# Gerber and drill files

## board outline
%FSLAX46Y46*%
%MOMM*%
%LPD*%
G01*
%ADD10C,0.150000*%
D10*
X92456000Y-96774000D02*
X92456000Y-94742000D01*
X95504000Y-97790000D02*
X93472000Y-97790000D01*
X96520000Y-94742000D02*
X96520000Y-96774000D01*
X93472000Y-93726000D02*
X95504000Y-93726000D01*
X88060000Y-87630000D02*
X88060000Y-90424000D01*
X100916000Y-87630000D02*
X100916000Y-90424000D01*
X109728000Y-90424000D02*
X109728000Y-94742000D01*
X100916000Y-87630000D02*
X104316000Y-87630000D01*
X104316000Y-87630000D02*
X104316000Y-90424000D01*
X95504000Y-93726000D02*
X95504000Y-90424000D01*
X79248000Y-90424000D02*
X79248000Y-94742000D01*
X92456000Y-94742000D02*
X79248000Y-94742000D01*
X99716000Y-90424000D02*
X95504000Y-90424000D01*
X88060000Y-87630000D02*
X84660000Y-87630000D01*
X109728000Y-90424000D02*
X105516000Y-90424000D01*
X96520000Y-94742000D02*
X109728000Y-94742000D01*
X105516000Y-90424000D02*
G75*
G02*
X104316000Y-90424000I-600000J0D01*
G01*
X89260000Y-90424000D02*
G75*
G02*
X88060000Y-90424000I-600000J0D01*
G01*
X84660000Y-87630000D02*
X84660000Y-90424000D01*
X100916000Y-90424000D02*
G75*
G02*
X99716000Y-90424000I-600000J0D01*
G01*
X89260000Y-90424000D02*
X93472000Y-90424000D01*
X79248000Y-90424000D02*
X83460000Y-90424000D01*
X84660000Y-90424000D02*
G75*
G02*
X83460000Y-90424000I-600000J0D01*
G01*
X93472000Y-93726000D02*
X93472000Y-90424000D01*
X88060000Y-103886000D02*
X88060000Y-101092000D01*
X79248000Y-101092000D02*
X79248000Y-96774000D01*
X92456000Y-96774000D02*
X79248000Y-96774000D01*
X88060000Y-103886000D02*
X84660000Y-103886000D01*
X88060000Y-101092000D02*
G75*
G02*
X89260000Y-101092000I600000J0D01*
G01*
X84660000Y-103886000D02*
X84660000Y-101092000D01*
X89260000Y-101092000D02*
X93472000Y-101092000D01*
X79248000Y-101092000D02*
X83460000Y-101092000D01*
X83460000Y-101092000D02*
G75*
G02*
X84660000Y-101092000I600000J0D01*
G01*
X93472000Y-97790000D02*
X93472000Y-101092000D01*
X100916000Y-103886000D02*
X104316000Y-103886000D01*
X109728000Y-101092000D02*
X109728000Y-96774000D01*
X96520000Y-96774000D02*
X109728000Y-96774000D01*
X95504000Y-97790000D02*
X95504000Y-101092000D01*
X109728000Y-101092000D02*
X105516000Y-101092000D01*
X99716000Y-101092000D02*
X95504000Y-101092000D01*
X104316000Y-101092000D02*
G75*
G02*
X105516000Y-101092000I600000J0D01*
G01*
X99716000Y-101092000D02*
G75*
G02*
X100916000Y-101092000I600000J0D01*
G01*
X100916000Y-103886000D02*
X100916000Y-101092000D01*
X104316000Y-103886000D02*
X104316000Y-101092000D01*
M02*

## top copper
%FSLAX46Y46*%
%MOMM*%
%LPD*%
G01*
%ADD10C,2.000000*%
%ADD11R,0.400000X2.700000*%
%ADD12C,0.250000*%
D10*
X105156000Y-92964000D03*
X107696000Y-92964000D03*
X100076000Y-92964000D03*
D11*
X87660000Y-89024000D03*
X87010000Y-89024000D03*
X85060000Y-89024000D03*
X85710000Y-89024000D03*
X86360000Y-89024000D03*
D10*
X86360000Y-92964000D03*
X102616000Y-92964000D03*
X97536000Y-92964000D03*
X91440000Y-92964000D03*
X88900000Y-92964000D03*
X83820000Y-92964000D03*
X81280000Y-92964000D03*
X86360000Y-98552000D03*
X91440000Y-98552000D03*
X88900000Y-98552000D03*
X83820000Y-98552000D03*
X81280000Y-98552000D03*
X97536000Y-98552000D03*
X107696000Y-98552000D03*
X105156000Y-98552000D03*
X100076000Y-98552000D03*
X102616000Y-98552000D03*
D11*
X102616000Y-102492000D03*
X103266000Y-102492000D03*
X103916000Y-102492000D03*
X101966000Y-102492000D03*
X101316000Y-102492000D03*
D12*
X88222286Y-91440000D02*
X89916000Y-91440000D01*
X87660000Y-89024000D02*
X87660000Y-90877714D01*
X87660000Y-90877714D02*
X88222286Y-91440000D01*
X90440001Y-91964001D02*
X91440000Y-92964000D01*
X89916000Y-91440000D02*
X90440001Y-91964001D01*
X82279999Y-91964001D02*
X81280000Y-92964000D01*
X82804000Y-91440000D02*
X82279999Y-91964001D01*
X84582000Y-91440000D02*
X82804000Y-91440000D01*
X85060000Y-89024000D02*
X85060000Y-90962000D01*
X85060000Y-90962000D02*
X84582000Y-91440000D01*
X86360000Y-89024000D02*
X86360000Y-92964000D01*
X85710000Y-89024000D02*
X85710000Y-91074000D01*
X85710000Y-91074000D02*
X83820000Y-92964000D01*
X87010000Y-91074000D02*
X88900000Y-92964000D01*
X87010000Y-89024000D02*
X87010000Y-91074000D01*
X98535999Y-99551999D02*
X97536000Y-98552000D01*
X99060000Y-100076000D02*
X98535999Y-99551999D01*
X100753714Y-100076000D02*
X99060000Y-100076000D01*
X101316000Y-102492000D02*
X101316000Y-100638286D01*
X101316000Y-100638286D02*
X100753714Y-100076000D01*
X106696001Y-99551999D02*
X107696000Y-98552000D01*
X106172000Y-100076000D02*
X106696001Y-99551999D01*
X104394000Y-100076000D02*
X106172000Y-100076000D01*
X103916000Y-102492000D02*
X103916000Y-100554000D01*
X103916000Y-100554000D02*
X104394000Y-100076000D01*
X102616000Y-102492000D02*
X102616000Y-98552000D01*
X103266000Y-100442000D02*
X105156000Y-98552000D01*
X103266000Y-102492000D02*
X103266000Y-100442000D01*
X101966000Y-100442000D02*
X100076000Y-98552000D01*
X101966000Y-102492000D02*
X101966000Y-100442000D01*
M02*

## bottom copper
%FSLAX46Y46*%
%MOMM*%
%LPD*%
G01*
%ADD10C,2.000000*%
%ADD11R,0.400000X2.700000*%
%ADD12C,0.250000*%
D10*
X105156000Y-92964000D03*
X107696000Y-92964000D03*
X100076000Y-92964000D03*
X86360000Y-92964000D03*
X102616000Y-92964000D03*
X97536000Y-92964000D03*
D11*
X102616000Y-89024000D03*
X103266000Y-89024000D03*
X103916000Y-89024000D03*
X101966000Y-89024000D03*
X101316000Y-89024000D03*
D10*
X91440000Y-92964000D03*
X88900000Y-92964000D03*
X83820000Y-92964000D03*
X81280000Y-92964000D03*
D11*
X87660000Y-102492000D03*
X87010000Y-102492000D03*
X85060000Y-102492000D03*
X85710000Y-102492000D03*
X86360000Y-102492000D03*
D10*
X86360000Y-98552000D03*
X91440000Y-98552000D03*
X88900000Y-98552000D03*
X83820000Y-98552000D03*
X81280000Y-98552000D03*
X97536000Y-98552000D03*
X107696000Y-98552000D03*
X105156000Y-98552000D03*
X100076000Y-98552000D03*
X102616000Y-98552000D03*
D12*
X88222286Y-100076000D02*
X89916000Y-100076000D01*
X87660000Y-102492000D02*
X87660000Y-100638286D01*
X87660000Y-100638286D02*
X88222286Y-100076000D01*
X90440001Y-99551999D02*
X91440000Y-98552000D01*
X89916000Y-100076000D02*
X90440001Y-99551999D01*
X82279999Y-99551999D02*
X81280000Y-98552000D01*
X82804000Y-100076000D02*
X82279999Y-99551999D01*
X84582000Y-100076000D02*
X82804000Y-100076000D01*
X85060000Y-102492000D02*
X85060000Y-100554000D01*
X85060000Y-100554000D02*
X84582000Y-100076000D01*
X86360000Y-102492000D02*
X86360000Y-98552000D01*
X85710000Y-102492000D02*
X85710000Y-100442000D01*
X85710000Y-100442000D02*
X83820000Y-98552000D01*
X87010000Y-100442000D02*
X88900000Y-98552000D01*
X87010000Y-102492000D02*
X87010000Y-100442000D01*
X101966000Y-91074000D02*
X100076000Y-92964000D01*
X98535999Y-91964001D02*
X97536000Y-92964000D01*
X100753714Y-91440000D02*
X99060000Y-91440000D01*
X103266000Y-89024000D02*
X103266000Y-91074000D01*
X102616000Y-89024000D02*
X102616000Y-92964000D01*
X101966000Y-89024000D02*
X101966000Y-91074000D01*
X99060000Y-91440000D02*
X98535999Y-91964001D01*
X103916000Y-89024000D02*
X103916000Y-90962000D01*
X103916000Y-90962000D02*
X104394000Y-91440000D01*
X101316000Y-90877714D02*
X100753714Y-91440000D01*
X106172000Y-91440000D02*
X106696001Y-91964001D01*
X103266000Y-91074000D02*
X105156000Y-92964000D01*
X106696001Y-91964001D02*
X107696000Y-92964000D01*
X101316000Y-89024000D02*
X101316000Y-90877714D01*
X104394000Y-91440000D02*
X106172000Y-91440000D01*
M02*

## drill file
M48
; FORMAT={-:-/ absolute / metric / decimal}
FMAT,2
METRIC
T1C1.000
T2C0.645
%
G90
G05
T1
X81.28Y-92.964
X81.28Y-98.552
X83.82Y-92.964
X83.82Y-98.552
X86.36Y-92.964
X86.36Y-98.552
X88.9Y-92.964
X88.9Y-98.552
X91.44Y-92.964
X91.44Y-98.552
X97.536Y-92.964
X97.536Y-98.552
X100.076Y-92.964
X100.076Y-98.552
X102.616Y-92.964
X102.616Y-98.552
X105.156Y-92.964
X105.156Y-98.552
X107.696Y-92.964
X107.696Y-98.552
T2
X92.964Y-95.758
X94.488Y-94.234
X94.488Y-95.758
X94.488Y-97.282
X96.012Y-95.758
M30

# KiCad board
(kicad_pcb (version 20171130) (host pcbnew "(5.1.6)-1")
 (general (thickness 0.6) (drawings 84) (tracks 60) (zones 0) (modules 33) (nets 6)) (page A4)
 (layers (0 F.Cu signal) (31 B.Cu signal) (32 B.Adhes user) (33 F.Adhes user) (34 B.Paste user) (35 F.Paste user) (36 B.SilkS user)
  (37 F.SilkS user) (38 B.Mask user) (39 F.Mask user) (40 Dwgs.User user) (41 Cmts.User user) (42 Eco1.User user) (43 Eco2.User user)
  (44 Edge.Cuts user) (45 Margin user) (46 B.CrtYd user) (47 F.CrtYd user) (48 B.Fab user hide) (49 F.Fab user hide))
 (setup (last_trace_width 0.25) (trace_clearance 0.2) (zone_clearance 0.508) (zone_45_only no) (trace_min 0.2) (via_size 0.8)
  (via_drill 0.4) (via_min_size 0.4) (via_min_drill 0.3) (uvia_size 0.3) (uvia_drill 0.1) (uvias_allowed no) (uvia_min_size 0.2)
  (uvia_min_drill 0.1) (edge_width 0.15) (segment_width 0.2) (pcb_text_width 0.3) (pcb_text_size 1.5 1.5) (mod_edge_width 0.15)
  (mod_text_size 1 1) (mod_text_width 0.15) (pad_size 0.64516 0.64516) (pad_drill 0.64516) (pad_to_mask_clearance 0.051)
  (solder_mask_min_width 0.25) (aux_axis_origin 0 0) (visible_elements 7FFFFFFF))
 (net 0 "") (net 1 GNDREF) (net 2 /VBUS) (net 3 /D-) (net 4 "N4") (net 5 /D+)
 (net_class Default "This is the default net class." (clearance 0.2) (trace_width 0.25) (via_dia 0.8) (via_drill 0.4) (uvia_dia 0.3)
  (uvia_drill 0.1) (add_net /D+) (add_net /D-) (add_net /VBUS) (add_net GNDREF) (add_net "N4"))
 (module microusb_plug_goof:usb (layer B.Cu) (at 86.3364 88.9 180)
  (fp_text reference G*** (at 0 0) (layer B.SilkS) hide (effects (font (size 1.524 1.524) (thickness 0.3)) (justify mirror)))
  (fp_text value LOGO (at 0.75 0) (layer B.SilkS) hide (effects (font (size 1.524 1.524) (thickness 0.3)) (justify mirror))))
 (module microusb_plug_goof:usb (layer F.Cu) (at 102.6396 88.9)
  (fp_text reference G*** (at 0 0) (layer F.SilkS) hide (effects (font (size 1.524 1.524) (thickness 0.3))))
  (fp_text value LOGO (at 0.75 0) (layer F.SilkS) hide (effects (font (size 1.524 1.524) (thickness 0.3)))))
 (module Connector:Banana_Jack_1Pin (layer F.Cu) (at 94.488 97.282)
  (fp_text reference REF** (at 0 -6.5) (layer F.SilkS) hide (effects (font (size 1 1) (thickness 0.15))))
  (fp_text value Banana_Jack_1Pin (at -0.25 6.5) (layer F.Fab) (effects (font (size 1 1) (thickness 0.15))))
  (pad "" np_thru_hole circle (at 0 0) (size 0.64516 0.64516) (drill 0.64516) (layers *.Cu *.Mask)))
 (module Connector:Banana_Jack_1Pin (layer F.Cu) (at 94.488 94.234)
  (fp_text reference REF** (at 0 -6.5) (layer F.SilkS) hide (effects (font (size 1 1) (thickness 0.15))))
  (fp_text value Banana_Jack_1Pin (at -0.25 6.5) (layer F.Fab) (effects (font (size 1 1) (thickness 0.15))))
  (pad "" np_thru_hole circle (at 0 0) (size 0.64516 0.64516) (drill 0.64516) (layers *.Cu *.Mask)))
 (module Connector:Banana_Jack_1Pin (layer F.Cu) (at 96.012 95.758)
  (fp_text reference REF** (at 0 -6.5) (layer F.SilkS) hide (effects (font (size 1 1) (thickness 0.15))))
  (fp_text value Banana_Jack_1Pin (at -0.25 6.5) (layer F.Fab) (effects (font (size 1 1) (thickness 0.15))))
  (pad "" np_thru_hole circle (at 0 0) (size 0.64516 0.64516) (drill 0.64516) (layers *.Cu *.Mask)))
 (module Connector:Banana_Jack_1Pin (layer F.Cu) (at 92.964 95.758)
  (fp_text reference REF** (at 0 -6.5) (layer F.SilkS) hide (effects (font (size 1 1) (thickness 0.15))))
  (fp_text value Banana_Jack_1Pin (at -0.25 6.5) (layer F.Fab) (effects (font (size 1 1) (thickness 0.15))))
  (pad "" np_thru_hole circle (at 0 0) (size 0.64516 0.64516) (drill 0.64516) (layers *.Cu *.Mask)))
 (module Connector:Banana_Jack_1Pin (layer F.Cu) (at 94.488 95.758)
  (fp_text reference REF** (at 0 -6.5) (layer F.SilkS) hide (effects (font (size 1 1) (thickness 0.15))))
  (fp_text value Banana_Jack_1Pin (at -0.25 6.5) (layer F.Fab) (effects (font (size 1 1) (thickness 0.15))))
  (pad "" np_thru_hole circle (at 0 0) (size 0.64516 0.64516) (drill 0.64516) (layers *.Cu *.Mask)))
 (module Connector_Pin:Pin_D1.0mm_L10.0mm (layer B.Cu) (at 105.156 92.964)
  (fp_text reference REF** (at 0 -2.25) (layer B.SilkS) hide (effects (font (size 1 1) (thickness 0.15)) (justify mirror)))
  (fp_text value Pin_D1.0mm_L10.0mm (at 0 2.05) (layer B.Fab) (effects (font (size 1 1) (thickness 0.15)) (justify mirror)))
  (pad 1 thru_hole circle (at 0 0) (size 2 2) (drill 1) (layers *.Cu *.Mask)))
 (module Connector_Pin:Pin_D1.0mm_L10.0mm (layer B.Cu) (at 107.696 92.964)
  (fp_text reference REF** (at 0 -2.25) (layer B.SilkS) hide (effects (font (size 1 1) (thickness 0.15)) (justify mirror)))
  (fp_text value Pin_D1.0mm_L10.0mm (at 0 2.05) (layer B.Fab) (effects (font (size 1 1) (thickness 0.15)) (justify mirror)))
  (pad 1 thru_hole circle (at 0 0) (size 2 2) (drill 1) (layers *.Cu *.Mask)))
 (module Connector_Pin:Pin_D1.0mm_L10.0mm (layer B.Cu) (at 100.076 92.964)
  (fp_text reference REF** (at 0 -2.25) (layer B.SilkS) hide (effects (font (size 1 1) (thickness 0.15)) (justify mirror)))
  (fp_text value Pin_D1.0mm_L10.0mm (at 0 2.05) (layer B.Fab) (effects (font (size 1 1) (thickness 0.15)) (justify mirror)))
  (pad 1 thru_hole circle (at 0 0) (size 2 2) (drill 1) (layers *.Cu *.Mask)))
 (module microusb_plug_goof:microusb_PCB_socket (layer F.Cu) (at 86.36 89.024)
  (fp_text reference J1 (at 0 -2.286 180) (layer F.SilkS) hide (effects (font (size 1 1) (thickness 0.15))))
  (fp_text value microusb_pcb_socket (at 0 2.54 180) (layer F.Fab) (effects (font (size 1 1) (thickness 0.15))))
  (pad 5 smd rect (at 1.3 0) (size 0.4 2.7) (layers F.Cu F.Paste F.Mask))
  (pad 4 smd rect (at 0.65 0) (size 0.4 2.7) (layers F.Cu F.Paste F.Mask))
  (pad 1 smd rect (at -1.3 0) (size 0.4 2.7) (layers F.Cu F.Paste F.Mask))
  (pad 2 smd rect (at -0.65 0) (size 0.4 2.7) (layers F.Cu F.Paste F.Mask))
  (pad 3 smd rect (at 0 0) (size 0.4 2.7) (layers F.Cu F.Paste F.Mask)))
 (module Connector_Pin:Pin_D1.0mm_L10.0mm (layer F.Cu) (at 86.36 92.964 180)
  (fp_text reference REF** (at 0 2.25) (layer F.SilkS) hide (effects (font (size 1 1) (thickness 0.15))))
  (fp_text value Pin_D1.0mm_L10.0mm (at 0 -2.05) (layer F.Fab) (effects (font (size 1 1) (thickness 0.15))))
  (pad 1 thru_hole circle (at 0 0 180) (size 2 2) (drill 1) (layers *.Cu *.Mask)))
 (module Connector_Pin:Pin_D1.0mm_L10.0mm (layer B.Cu) (at 102.616 92.964)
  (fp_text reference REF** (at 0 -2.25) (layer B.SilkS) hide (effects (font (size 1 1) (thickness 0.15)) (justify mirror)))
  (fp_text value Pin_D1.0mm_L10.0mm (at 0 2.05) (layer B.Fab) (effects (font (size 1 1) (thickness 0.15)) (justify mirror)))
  (pad 1 thru_hole circle (at 0 0) (size 2 2) (drill 1) (layers *.Cu *.Mask)))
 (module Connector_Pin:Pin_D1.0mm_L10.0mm (layer B.Cu) (at 97.536 92.964)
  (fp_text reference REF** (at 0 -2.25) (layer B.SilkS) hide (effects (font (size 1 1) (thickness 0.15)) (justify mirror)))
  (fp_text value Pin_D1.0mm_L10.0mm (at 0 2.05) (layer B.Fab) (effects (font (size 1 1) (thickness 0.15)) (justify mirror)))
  (pad 1 thru_hole circle (at 0 0) (size 2 2) (drill 1) (layers *.Cu *.Mask)))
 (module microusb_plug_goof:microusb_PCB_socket (layer B.Cu) (at 102.616 89.024 180)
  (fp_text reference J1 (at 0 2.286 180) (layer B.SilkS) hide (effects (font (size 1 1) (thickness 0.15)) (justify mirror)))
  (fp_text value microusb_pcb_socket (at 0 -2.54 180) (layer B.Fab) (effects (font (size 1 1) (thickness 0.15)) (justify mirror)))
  (pad 3 smd rect (at 0 0 180) (size 0.4 2.7) (layers B.Cu B.Paste B.Mask))
  (pad 2 smd rect (at -0.65 0 180) (size 0.4 2.7) (layers B.Cu B.Paste B.Mask))
  (pad 1 smd rect (at -1.3 0 180) (size 0.4 2.7) (layers B.Cu B.Paste B.Mask))
  (pad 4 smd rect (at 0.65 0 180) (size 0.4 2.7) (layers B.Cu B.Paste B.Mask))
  (pad 5 smd rect (at 1.3 0 180) (size 0.4 2.7) (layers B.Cu B.Paste B.Mask)))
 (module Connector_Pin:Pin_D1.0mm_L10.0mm (layer F.Cu) (at 91.44 92.964 180)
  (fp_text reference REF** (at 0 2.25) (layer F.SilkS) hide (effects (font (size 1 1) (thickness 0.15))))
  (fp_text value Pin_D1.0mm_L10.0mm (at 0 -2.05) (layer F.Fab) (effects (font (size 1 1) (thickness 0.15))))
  (pad 1 thru_hole circle (at 0 0 180) (size 2 2) (drill 1) (layers *.Cu *.Mask)))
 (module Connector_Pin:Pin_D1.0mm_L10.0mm (layer F.Cu) (at 88.9 92.964 180)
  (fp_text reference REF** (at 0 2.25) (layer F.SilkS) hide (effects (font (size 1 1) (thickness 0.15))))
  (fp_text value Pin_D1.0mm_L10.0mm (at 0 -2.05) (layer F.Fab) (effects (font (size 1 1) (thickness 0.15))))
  (pad 1 thru_hole circle (at 0 0 180) (size 2 2) (drill 1) (layers *.Cu *.Mask)))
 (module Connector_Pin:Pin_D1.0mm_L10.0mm (layer F.Cu) (at 83.82 92.964 180)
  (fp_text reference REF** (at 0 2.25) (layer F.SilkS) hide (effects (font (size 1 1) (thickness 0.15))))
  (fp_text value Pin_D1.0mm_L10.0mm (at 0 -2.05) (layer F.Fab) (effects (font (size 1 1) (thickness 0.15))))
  (pad 1 thru_hole circle (at 0 0 180) (size 2 2) (drill 1) (layers *.Cu *.Mask)))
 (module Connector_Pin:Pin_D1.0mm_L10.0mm (layer F.Cu) (at 81.28 92.964 180)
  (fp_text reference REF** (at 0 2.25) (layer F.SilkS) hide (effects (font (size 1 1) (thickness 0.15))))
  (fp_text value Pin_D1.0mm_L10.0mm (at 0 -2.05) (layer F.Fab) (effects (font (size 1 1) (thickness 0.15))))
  (pad 1 thru_hole circle (at 0 0 180) (size 2 2) (drill 1) (layers *.Cu *.Mask)))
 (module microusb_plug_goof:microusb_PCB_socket (layer B.Cu) (at 86.36 102.492)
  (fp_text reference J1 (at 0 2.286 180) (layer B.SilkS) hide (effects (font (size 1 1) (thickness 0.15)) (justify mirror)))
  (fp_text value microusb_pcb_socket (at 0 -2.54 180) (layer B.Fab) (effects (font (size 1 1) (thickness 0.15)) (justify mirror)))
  (pad 5 smd rect (at 1.3 0) (size 0.4 2.7) (layers B.Cu B.Paste B.Mask))
  (pad 4 smd rect (at 0.65 0) (size 0.4 2.7) (layers B.Cu B.Paste B.Mask))
  (pad 1 smd rect (at -1.3 0) (size 0.4 2.7) (layers B.Cu B.Paste B.Mask))
  (pad 2 smd rect (at -0.65 0) (size 0.4 2.7) (layers B.Cu B.Paste B.Mask))
  (pad 3 smd rect (at 0 0) (size 0.4 2.7) (layers B.Cu B.Paste B.Mask)))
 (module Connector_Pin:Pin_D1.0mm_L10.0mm (layer B.Cu) (at 86.36 98.552 180)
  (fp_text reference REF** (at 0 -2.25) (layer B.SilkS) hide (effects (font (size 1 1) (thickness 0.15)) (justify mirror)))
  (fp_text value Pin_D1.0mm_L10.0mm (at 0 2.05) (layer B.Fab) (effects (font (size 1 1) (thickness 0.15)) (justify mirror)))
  (pad 1 thru_hole circle (at 0 0 180) (size 2 2) (drill 1) (layers *.Cu *.Mask)))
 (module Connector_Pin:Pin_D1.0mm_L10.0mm (layer B.Cu) (at 91.44 98.552 180)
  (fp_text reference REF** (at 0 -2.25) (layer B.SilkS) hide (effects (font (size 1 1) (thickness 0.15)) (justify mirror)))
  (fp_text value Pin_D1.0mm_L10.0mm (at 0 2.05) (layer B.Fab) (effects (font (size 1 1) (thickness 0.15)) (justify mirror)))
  (pad 1 thru_hole circle (at 0 0 180) (size 2 2) (drill 1) (layers *.Cu *.Mask)))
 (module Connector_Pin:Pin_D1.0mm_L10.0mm (layer B.Cu) (at 88.9 98.552 180)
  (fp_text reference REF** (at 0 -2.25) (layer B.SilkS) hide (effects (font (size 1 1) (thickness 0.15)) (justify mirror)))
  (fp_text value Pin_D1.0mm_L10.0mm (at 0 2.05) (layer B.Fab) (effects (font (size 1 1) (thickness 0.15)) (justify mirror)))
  (pad 1 thru_hole circle (at 0 0 180) (size 2 2) (drill 1) (layers *.Cu *.Mask)))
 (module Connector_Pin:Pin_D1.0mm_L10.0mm (layer B.Cu) (at 83.82 98.552 180)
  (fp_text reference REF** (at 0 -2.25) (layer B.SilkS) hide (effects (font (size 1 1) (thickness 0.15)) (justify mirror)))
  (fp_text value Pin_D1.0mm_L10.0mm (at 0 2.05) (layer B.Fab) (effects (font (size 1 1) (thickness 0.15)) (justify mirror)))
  (pad 1 thru_hole circle (at 0 0 180) (size 2 2) (drill 1) (layers *.Cu *.Mask)))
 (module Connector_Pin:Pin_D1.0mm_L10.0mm (layer B.Cu) (at 81.28 98.552 180)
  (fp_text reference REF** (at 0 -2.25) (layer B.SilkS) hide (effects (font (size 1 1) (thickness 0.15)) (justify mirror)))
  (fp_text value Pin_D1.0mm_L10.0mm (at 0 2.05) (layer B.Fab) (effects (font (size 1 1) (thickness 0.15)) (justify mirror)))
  (pad 1 thru_hole circle (at 0 0 180) (size 2 2) (drill 1) (layers *.Cu *.Mask)))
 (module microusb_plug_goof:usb (layer F.Cu) (at 86.36 102.616 180)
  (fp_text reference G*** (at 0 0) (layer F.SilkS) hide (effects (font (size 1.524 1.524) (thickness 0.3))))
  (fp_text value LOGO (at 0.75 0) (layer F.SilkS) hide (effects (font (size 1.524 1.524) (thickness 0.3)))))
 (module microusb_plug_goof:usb (layer B.Cu) (at 102.616 102.616)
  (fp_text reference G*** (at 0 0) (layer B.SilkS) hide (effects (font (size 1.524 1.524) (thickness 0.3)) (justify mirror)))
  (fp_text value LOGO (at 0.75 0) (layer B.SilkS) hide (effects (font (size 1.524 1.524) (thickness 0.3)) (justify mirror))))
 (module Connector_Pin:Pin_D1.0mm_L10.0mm (layer F.Cu) (at 97.536 98.552)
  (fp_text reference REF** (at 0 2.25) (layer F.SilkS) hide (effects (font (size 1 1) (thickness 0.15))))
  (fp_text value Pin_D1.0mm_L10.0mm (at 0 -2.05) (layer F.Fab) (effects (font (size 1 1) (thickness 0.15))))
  (pad 1 thru_hole circle (at 0 0) (size 2 2) (drill 1) (layers *.Cu *.Mask) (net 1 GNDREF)))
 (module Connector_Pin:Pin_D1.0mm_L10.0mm (layer F.Cu) (at 107.696 98.552)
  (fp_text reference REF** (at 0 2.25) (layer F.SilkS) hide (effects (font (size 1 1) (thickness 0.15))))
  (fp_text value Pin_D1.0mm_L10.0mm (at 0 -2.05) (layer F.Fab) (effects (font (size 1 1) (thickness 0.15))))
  (pad 1 thru_hole circle (at 0 0) (size 2 2) (drill 1) (layers *.Cu *.Mask) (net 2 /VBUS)))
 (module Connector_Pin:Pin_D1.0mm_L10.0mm (layer F.Cu) (at 105.156 98.552)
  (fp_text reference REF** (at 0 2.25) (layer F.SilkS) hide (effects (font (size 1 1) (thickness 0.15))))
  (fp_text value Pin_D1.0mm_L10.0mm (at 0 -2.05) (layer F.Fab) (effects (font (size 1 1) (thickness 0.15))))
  (pad 1 thru_hole circle (at 0 0) (size 2 2) (drill 1) (layers *.Cu *.Mask) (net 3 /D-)))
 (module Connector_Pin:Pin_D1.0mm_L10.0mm (layer F.Cu) (at 100.076 98.552)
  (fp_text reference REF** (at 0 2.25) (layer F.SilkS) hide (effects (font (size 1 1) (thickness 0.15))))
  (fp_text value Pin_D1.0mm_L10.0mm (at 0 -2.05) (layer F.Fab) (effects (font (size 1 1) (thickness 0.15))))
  (pad 1 thru_hole circle (at 0 0) (size 2 2) (drill 1) (layers *.Cu *.Mask) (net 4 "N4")))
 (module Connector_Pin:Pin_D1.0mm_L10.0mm (layer F.Cu) (at 102.616 98.552)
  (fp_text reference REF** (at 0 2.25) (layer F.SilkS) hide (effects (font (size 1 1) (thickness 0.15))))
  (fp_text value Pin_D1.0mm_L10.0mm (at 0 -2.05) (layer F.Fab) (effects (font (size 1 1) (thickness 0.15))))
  (pad 1 thru_hole circle (at 0 0) (size 2 2) (drill 1) (layers *.Cu *.Mask) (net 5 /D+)))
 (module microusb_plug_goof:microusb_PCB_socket (layer F.Cu) (at 102.616 102.492 180)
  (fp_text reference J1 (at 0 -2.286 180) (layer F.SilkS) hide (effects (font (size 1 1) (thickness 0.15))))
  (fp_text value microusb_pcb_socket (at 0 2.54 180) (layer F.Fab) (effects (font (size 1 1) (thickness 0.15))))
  (pad 3 smd rect (at 0 0 180) (size 0.4 2.7) (layers F.Cu F.Paste F.Mask) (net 5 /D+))
  (pad 2 smd rect (at -0.65 0 180) (size 0.4 2.7) (layers F.Cu F.Paste F.Mask) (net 3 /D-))
  (pad 1 smd rect (at -1.3 0 180) (size 0.4 2.7) (layers F.Cu F.Paste F.Mask) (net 2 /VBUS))
  (pad 4 smd rect (at 0.65 0 180) (size 0.4 2.7) (layers F.Cu F.Paste F.Mask) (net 4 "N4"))
  (pad 5 smd rect (at 1.3 0 180) (size 0.4 2.7) (layers F.Cu F.Paste F.Mask) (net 1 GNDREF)))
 (gr_line (start 92.456 96.774) (end 92.456 94.742) (layer Edge.Cuts) (width 0.15))
 (gr_line (start 95.504 97.79) (end 93.472 97.79) (layer Edge.Cuts) (width 0.15))
 (gr_line (start 96.52 94.742) (end 96.52 96.774) (layer Edge.Cuts) (width 0.15))
 (gr_line (start 93.472 93.726) (end 95.504 93.726) (layer Edge.Cuts) (width 0.15))
 (gr_line (start 88.06 87.63) (end 88.06 90.424) (layer Edge.Cuts) (width 0.15))
 (gr_line (start 100.916 87.63) (end 100.916 90.424) (layer Edge.Cuts) (width 0.15))
 (gr_line (start 109.728 90.424) (end 109.728 94.742) (layer Edge.Cuts) (width 0.15))
 (gr_line (start 100.916 87.63) (end 104.316 87.63) (layer Edge.Cuts) (width 0.15))
 (gr_line (start 104.316 87.63) (end 104.316 90.424) (layer Edge.Cuts) (width 0.15))
 (gr_line (start 95.504 93.726) (end 95.504 90.424) (layer Edge.Cuts) (width 0.15))
 (gr_line (start 79.248 90.424) (end 79.248 94.742) (layer Edge.Cuts) (width 0.15))
 (gr_line (start 92.456 94.742) (end 79.248 94.742) (layer Edge.Cuts) (width 0.15))
 (gr_line (start 99.716 90.424) (end 95.504 90.424) (layer Edge.Cuts) (width 0.15))
 (gr_line (start 88.06 87.63) (end 84.66 87.63) (layer Edge.Cuts) (width 0.15))
 (gr_line (start 109.728 90.424) (end 105.516 90.424) (layer Edge.Cuts) (width 0.15))
 (gr_line (start 96.52 94.742) (end 109.728 94.742) (layer Edge.Cuts) (width 0.15))
 (gr_arc (start 104.916 90.424) (end 104.316 90.424) (angle -180) (layer Edge.Cuts) (width 0.15))
 (gr_arc (start 88.66 90.424) (end 88.06 90.424) (angle -180) (layer Edge.Cuts) (width 0.15))
 (gr_line (start 84.66 87.63) (end 84.66 90.424) (layer Edge.Cuts) (width 0.15))
 (gr_arc (start 100.316 90.424) (end 100.916 90.424) (angle 180) (layer Edge.Cuts) (width 0.15))
 (gr_line (start 89.26 90.424) (end 93.472 90.424) (layer Edge.Cuts) (width 0.15))
 (gr_line (start 79.248 90.424) (end 83.46 90.424) (layer Edge.Cuts) (width 0.15))
 (gr_arc (start 84.06 90.424) (end 84.66 90.424) (angle 180) (layer Edge.Cuts) (width 0.15))
 (gr_line (start 93.472 93.726) (end 93.472 90.424) (layer Edge.Cuts) (width 0.15))
 (gr_line (start 88.06 103.886) (end 88.06 101.092) (layer Edge.Cuts) (width 0.15))
 (gr_line (start 79.248 101.092) (end 79.248 96.774) (layer Edge.Cuts) (width 0.15))
 (gr_line (start 92.456 96.774) (end 79.248 96.774) (layer Edge.Cuts) (width 0.15))
 (gr_line (start 88.06 103.886) (end 84.66 103.886) (layer Edge.Cuts) (width 0.15))
 (gr_arc (start 88.66 101.092) (end 88.06 101.092) (angle 180) (layer Edge.Cuts) (width 0.15))
 (gr_line (start 84.66 103.886) (end 84.66 101.092) (layer Edge.Cuts) (width 0.15))
 (gr_line (start 89.26 101.092) (end 93.472 101.092) (layer Edge.Cuts) (width 0.15))
 (gr_line (start 79.248 101.092) (end 83.46 101.092) (layer Edge.Cuts) (width 0.15))
 (gr_arc (start 84.06 101.092) (end 84.66 101.092) (angle -180) (layer Edge.Cuts) (width 0.15))
 (gr_line (start 93.472 97.79) (end 93.472 101.092) (layer Edge.Cuts) (width 0.15))
 (gr_line (start 100.916 103.886) (end 104.316 103.886) (layer Edge.Cuts) (width 0.15))
 (gr_line (start 109.728 101.092) (end 109.728 96.774) (layer Edge.Cuts) (width 0.15))
 (gr_line (start 96.52 96.774) (end 109.728 96.774) (layer Edge.Cuts) (width 0.15))
 (gr_line (start 95.504 97.79) (end 95.504 101.092) (layer Edge.Cuts) (width 0.15))
 (gr_line (start 109.728 101.092) (end 105.516 101.092) (layer Edge.Cuts) (width 0.15))
 (gr_line (start 99.716 101.092) (end 95.504 101.092) (layer Edge.Cuts) (width 0.15))
 (gr_arc (start 104.916 101.092) (end 104.316 101.092) (angle 180) (layer Edge.Cuts) (width 0.15))
 (gr_arc (start 100.316 101.092) (end 100.916 101.092) (angle -180) (layer Edge.Cuts) (width 0.15))
 (gr_line (start 100.916 103.886) (end 100.916 101.092) (layer Edge.Cuts) (width 0.15))
 (gr_line (start 104.316 103.886) (end 104.316 101.092) (layer Edge.Cuts) (width 0.15))
 (segment (start 88.222286 100.076) (end 89.916 100.076) (width 0.25) (layer B.Cu) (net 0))
 (segment (start 87.66 102.492) (end 87.66 100.638286) (width 0.25) (layer B.Cu) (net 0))
 (segment (start 87.66 100.638286) (end 88.222286 100.076) (width 0.25) (layer B.Cu) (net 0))
 (segment (start 90.440001 99.551999) (end 91.44 98.552) (width 0.25) (layer B.Cu) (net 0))
 (segment (start 89.916 100.076) (end 90.440001 99.551999) (width 0.25) (layer B.Cu) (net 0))
 (segment (start 82.279999 99.551999) (end 81.28 98.552) (width 0.25) (layer B.Cu) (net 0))
 (segment (start 82.804 100.076) (end 82.279999 99.551999) (width 0.25) (layer B.Cu) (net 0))
 (segment (start 84.582 100.076) (end 82.804 100.076) (width 0.25) (layer B.Cu) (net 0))
 (segment (start 85.06 102.492) (end 85.06 100.554) (width 0.25) (layer B.Cu) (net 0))
 (segment (start 85.06 100.554) (end 84.582 100.076) (width 0.25) (layer B.Cu) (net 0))
 (segment (start 86.36 102.492) (end 86.36 98.552) (width 0.25) (layer B.Cu) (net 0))
 (segment (start 85.71 102.492) (end 85.71 100.442) (width 0.25) (layer B.Cu) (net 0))
 (segment (start 85.71 100.442) (end 83.82 98.552) (width 0.25) (layer B.Cu) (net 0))
 (segment (start 87.01 100.442) (end 88.9 98.552) (width 0.25) (layer B.Cu) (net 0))
 (segment (start 87.01 102.492) (end 87.01 100.442) (width 0.25) (layer B.Cu) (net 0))
 (segment (start 101.966 91.074) (end 100.076 92.964) (width 0.25) (layer B.Cu) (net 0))
 (segment (start 98.535999 91.964001) (end 97.536 92.964) (width 0.25) (layer B.Cu) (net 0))
 (segment (start 100.753714 91.44) (end 99.06 91.44) (width 0.25) (layer B.Cu) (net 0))
 (segment (start 103.266 89.024) (end 103.266 91.074) (width 0.25) (layer B.Cu) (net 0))
 (segment (start 102.616 89.024) (end 102.616 92.964) (width 0.25) (layer B.Cu) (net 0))
 (segment (start 101.966 89.024) (end 101.966 91.074) (width 0.25) (layer B.Cu) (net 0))
 (segment (start 99.06 91.44) (end 98.535999 91.964001) (width 0.25) (layer B.Cu) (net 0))
 (segment (start 103.916 89.024) (end 103.916 90.962) (width 0.25) (layer B.Cu) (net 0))
 (segment (start 103.916 90.962) (end 104.394 91.44) (width 0.25) (layer B.Cu) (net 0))
 (segment (start 101.316 90.877714) (end 100.753714 91.44) (width 0.25) (layer B.Cu) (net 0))
 (segment (start 106.172 91.44) (end 106.696001 91.964001) (width 0.25) (layer B.Cu) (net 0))
 (segment (start 103.266 91.074) (end 105.156 92.964) (width 0.25) (layer B.Cu) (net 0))
 (segment (start 106.696001 91.964001) (end 107.696 92.964) (width 0.25) (layer B.Cu) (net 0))
 (segment (start 101.316 89.024) (end 101.316 90.877714) (width 0.25) (layer B.Cu) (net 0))
 (segment (start 104.394 91.44) (end 106.172 91.44) (width 0.25) (layer B.Cu) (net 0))
 (segment (start 88.222286 91.44) (end 89.916 91.44) (width 0.25) (layer F.Cu) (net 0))
 (segment (start 87.66 89.024) (end 87.66 90.877714) (width 0.25) (layer F.Cu) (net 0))
 (segment (start 87.66 90.877714) (end 88.222286 91.44) (width 0.25) (layer F.Cu) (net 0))
 (segment (start 90.440001 91.964001) (end 91.44 92.964) (width 0.25) (layer F.Cu) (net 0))
 (segment (start 89.916 91.44) (end 90.440001 91.964001) (width 0.25) (layer F.Cu) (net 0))
 (segment (start 82.279999 91.964001) (end 81.28 92.964) (width 0.25) (layer F.Cu) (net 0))
 (segment (start 82.804 91.44) (end 82.279999 91.964001) (width 0.25) (layer F.Cu) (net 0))
 (segment (start 84.582 91.44) (end 82.804 91.44) (width 0.25) (layer F.Cu) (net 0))
 (segment (start 85.06 89.024) (end 85.06 90.962) (width 0.25) (layer F.Cu) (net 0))
 (segment (start 85.06 90.962) (end 84.582 91.44) (width 0.25) (layer F.Cu) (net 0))
 (segment (start 86.36 89.024) (end 86.36 92.964) (width 0.25) (layer F.Cu) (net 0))
 (segment (start 85.71 89.024) (end 85.71 91.074) (width 0.25) (layer F.Cu) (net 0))
 (segment (start 85.71 91.074) (end 83.82 92.964) (width 0.25) (layer F.Cu) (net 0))
 (segment (start 87.01 91.074) (end 88.9 92.964) (width 0.25) (layer F.Cu) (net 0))
 (segment (start 87.01 89.024) (end 87.01 91.074) (width 0.25) (layer F.Cu) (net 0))
 (segment (start 98.535999 99.551999) (end 97.536 98.552) (width 0.25) (layer F.Cu) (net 1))
 (segment (start 99.06 100.076) (end 98.535999 99.551999) (width 0.25) (layer F.Cu) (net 1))
 (segment (start 100.753714 100.076) (end 99.06 100.076) (width 0.25) (layer F.Cu) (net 1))
 (segment (start 101.316 102.492) (end 101.316 100.638286) (width 0.25) (layer F.Cu) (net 1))
 (segment (start 101.316 100.638286) (end 100.753714 100.076) (width 0.25) (layer F.Cu) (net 1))
 (segment (start 106.696001 99.551999) (end 107.696 98.552) (width 0.25) (layer F.Cu) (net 2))
 (segment (start 106.172 100.076) (end 106.696001 99.551999) (width 0.25) (layer F.Cu) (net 2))
 (segment (start 104.394 100.076) (end 106.172 100.076) (width 0.25) (layer F.Cu) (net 2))
 (segment (start 103.916 102.492) (end 103.916 100.554) (width 0.25) (layer F.Cu) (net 2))
 (segment (start 103.916 100.554) (end 104.394 100.076) (width 0.25) (layer F.Cu) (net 2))
 (segment (start 102.616 102.492) (end 102.616 98.552) (width 0.25) (layer F.Cu) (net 5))
 (segment (start 103.266 100.442) (end 105.156 98.552) (width 0.25) (layer F.Cu) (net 3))
 (segment (start 103.266 102.492) (end 103.266 100.442) (width 0.25) (layer F.Cu) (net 3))
 (segment (start 101.966 100.442) (end 100.076 98.552) (width 0.25) (layer F.Cu) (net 4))
 (segment (start 101.966 102.492) (end 101.966 100.442) (width 0.25) (layer F.Cu) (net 4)))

